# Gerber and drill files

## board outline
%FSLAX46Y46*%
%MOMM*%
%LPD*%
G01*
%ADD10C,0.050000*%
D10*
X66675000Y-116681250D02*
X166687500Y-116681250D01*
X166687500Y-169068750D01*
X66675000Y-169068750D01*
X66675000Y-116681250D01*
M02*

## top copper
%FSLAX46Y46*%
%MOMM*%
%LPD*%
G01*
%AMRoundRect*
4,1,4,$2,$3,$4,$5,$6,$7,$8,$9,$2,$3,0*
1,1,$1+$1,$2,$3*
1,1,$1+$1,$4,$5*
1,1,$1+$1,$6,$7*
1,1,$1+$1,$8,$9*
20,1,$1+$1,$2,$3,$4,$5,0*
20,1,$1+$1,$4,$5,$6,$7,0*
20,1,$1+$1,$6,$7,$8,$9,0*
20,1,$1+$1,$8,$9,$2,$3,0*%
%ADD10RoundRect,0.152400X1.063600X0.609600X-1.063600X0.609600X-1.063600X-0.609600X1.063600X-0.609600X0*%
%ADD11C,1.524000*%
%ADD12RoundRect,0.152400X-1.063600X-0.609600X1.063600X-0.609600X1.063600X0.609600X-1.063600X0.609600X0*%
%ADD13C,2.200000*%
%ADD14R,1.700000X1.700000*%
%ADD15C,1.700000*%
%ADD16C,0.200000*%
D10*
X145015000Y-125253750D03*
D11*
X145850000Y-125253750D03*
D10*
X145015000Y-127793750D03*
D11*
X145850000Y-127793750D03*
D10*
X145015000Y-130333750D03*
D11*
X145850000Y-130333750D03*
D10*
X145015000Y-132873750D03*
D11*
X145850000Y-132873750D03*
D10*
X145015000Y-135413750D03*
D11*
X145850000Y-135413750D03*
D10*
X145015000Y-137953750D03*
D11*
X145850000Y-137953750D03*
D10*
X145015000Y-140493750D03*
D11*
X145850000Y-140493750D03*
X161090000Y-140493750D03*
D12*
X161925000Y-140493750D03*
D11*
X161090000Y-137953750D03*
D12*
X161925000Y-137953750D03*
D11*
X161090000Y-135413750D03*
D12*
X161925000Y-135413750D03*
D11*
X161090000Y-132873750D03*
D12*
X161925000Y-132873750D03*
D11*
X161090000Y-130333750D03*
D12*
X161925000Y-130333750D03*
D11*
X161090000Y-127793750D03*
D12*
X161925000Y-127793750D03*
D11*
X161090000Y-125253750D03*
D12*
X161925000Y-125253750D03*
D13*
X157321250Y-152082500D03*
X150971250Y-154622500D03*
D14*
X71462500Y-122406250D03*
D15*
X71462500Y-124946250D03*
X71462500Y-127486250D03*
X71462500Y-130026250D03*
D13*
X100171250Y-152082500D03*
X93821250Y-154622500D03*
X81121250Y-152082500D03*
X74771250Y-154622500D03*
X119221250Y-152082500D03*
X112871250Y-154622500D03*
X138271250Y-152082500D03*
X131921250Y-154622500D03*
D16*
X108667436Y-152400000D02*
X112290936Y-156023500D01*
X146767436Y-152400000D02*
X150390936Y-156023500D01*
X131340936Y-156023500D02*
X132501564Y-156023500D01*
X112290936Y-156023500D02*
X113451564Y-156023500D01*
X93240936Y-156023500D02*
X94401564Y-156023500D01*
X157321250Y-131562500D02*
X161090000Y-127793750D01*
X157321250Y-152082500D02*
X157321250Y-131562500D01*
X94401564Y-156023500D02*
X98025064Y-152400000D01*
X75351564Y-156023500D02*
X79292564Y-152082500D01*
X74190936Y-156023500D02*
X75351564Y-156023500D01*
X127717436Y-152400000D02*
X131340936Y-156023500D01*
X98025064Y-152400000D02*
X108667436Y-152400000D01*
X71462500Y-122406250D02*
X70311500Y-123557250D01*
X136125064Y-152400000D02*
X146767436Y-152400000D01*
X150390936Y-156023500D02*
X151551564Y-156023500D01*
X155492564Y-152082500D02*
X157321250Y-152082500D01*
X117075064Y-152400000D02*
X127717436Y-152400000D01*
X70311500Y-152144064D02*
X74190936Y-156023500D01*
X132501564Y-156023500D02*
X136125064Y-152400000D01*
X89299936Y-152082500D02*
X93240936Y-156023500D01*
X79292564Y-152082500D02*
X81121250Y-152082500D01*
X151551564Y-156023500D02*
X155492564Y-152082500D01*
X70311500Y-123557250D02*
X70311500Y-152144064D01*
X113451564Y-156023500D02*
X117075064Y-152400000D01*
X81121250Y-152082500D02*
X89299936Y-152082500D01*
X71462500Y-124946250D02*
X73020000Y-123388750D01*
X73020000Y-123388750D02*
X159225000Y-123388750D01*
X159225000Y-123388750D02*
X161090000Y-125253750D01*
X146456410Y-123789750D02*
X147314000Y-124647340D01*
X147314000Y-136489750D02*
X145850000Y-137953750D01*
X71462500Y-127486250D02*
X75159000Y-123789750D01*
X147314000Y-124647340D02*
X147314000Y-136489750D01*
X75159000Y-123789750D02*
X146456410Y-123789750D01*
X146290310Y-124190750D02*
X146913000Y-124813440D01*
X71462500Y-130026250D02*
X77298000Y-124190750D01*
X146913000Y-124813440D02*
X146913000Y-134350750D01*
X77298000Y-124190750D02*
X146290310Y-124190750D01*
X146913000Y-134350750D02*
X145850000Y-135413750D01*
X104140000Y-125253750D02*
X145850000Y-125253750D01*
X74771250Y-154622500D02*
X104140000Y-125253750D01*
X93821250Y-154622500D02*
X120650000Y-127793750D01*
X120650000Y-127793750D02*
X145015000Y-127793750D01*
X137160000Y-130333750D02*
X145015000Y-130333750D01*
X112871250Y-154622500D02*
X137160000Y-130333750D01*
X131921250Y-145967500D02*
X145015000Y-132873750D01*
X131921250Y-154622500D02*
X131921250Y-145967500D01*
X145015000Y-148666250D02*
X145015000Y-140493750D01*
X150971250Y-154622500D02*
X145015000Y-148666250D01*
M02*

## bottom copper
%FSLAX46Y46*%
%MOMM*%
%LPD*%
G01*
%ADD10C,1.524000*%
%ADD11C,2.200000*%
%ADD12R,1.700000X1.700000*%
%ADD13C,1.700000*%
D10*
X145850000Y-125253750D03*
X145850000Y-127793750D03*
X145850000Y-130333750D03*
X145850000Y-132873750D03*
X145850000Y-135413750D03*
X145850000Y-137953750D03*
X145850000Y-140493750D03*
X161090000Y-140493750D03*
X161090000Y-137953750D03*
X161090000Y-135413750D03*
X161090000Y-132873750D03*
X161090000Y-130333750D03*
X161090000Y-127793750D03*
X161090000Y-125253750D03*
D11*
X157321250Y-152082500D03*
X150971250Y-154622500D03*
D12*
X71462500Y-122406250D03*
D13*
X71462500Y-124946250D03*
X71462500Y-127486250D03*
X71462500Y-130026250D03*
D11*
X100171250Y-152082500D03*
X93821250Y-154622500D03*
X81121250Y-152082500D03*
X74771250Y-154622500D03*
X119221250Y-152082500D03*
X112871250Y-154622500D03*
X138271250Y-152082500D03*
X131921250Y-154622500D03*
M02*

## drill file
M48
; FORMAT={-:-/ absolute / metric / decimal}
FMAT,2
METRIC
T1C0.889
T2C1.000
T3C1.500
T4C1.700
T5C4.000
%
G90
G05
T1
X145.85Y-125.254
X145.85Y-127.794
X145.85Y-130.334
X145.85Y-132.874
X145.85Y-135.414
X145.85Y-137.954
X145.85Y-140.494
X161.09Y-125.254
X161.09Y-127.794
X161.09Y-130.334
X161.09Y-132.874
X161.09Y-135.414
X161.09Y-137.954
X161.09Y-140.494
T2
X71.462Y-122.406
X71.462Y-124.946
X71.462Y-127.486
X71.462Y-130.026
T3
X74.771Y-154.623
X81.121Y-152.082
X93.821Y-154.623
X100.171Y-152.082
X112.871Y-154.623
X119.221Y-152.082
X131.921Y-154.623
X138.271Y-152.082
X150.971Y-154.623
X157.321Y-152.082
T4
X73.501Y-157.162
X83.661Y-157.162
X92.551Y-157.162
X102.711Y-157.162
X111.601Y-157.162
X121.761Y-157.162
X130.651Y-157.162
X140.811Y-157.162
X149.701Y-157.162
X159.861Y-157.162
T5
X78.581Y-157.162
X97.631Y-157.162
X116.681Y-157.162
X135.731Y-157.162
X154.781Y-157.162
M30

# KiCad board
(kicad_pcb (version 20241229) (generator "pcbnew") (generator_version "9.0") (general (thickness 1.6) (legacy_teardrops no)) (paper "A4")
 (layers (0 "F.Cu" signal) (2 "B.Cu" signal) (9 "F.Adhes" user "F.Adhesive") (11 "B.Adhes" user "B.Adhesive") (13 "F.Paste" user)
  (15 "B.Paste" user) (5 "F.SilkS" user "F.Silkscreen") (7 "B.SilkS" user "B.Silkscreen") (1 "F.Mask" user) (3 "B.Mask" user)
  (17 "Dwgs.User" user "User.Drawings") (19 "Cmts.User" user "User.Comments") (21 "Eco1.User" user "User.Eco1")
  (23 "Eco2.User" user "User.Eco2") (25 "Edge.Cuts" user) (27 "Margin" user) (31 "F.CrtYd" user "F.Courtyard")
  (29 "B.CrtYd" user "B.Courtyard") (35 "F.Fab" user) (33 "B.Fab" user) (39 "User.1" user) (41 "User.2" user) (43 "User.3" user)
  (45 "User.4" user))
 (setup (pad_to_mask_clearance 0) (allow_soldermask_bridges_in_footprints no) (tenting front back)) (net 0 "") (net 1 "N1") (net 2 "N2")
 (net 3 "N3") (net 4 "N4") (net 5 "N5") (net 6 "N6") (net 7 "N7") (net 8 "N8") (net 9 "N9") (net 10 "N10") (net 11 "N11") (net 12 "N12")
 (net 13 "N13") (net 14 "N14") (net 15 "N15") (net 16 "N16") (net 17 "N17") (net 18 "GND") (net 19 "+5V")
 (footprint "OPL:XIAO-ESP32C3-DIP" (layer "F.Cu") (at 153.59 132.87375)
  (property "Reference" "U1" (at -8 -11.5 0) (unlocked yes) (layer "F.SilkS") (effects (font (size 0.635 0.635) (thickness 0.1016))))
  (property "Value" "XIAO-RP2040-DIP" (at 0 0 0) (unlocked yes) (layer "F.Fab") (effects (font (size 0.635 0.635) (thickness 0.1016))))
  (pad "1" smd roundrect (at -8.575 -7.62 180) (size 2.432 1.524) (layers "F.Cu" "F.Mask") (roundrect_rratio 0.1) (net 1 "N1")
   (thermal_bridge_angle 45))
  (pad "1" thru_hole circle (at -7.74 -7.62 180) (size 1.524 1.524) (drill 0.889) (layers "*.Cu" "*.Mask") (remove_unused_layers no)
   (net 1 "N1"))
  (pad "2" smd roundrect (at -8.575 -5.08 180) (size 2.432 1.524) (layers "F.Cu" "F.Mask") (roundrect_rratio 0.1) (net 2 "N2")
   (thermal_bridge_angle 45))
  (pad "2" thru_hole circle (at -7.74 -5.08 180) (size 1.524 1.524) (drill 0.889) (layers "*.Cu" "*.Mask") (remove_unused_layers no)
   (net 2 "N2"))
  (pad "3" smd roundrect (at -8.575 -2.54 180) (size 2.432 1.524) (layers "F.Cu" "F.Mask") (roundrect_rratio 0.1) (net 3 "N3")
   (thermal_bridge_angle 45))
  (pad "3" thru_hole circle (at -7.74 -2.54 180) (size 1.524 1.524) (drill 0.889) (layers "*.Cu" "*.Mask") (remove_unused_layers no)
   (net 3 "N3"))
  (pad "4" smd roundrect (at -8.575 0 180) (size 2.432 1.524) (layers "F.Cu" "F.Mask") (roundrect_rratio 0.1) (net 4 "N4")
   (thermal_bridge_angle 45))
  (pad "4" thru_hole circle (at -7.74 0 180) (size 1.524 1.524) (drill 0.889) (layers "*.Cu" "*.Mask") (remove_unused_layers no)
   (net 4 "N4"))
  (pad "5" smd roundrect (at -8.575 2.54 180) (size 2.432 1.524) (layers "F.Cu" "F.Mask") (roundrect_rratio 0.1) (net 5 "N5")
   (thermal_bridge_angle 45))
  (pad "5" thru_hole circle (at -7.74 2.54 180) (size 1.524 1.524) (drill 0.889) (layers "*.Cu" "*.Mask") (remove_unused_layers no)
   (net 5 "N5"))
  (pad "6" smd roundrect (at -8.575 5.08 180) (size 2.432 1.524) (layers "F.Cu" "F.Mask") (roundrect_rratio 0.1) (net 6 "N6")
   (thermal_bridge_angle 45))
  (pad "6" thru_hole circle (at -7.74 5.08 180) (size 1.524 1.524) (drill 0.889) (layers "*.Cu" "*.Mask") (remove_unused_layers no)
   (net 6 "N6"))
  (pad "7" smd roundrect (at -8.575 7.62 180) (size 2.432 1.524) (layers "F.Cu" "F.Mask") (roundrect_rratio 0.1) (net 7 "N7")
   (thermal_bridge_angle 45))
  (pad "7" thru_hole circle (at -7.74 7.62 180) (size 1.524 1.524) (drill 0.889) (layers "*.Cu" "*.Mask") (remove_unused_layers no)
   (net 7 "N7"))
  (pad "8" thru_hole circle (at 7.5 7.62) (size 1.524 1.524) (drill 0.889) (layers "*.Cu" "*.Mask") (remove_unused_layers no) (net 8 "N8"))
  (pad "8" smd roundrect (at 8.335 7.62) (size 2.432 1.524) (layers "F.Cu" "F.Mask") (roundrect_rratio 0.1) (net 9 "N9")
   (thermal_bridge_angle 45))
  (pad "9" thru_hole circle (at 7.5 5.08) (size 1.524 1.524) (drill 0.889) (layers "*.Cu" "*.Mask") (remove_unused_layers no) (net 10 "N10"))
  (pad "9" smd roundrect (at 8.335 5.08) (size 2.432 1.524) (layers "F.Cu" "F.Mask") (roundrect_rratio 0.1) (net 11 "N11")
   (thermal_bridge_angle 45))
  (pad "10" thru_hole circle (at 7.5 2.54) (size 1.524 1.524) (drill 0.889) (layers "*.Cu" "*.Mask") (remove_unused_layers no)
   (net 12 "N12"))
  (pad "10" smd roundrect (at 8.335 2.54) (size 2.432 1.524) (layers "F.Cu" "F.Mask") (roundrect_rratio 0.1) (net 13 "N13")
   (thermal_bridge_angle 45))
  (pad "11" thru_hole circle (at 7.5 0) (size 1.524 1.524) (drill 0.889) (layers "*.Cu" "*.Mask") (remove_unused_layers no) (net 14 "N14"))
  (pad "11" smd roundrect (at 8.335 0) (size 2.432 1.524) (layers "F.Cu" "F.Mask") (roundrect_rratio 0.1) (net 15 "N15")
   (thermal_bridge_angle 45))
  (pad "12" thru_hole circle (at 7.5 -2.54) (size 1.524 1.524) (drill 0.889) (layers "*.Cu" "*.Mask") (remove_unused_layers no)
   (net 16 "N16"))
  (pad "12" smd roundrect (at 8.335 -2.54) (size 2.432 1.524) (layers "F.Cu" "F.Mask") (roundrect_rratio 0.1) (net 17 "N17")
   (thermal_bridge_angle 45))
  (pad "13" thru_hole circle (at 7.5 -5.08) (size 1.524 1.524) (drill 0.889) (layers "*.Cu" "*.Mask") (remove_unused_layers no)
   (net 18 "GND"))
  (pad "13" smd roundrect (at 8.335 -5.08) (size 2.432 1.524) (layers "F.Cu" "F.Mask") (roundrect_rratio 0.1) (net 18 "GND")
   (thermal_bridge_angle 45))
  (pad "14" thru_hole circle (at 7.5 -7.62) (size 1.524 1.524) (drill 0.889) (layers "*.Cu" "*.Mask") (remove_unused_layers no)
   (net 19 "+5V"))
  (pad "14" smd roundrect (at 8.335 -7.62) (size 2.432 1.524) (layers "F.Cu" "F.Mask") (roundrect_rratio 0.1) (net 19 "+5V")
   (thermal_bridge_angle 45)))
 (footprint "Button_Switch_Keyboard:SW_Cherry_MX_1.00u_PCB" (layer "F.Cu") (at 157.32125 152.0825)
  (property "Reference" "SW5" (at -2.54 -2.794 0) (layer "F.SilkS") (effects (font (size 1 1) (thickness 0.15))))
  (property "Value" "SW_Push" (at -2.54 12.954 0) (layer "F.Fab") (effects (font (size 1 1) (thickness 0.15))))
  (pad "" np_thru_hole circle (at -7.62 5.08) (size 1.7 1.7) (drill 1.7) (layers "*.Cu" "*.Mask"))
  (pad "" np_thru_hole circle (at -2.54 5.08) (size 4 4) (drill 4) (layers "*.Cu" "*.Mask"))
  (pad "" np_thru_hole circle (at 2.54 5.08) (size 1.7 1.7) (drill 1.7) (layers "*.Cu" "*.Mask"))
  (pad "1" thru_hole circle (at 0 0) (size 2.2 2.2) (drill 1.5) (layers "*.Cu" "*.Mask") (remove_unused_layers no) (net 18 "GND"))
  (pad "2" thru_hole circle (at -6.35 2.54) (size 2.2 2.2) (drill 1.5) (layers "*.Cu" "*.Mask") (remove_unused_layers no) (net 7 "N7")))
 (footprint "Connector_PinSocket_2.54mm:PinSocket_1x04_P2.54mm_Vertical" (layer "F.Cu") (at 71.4625 122.40625)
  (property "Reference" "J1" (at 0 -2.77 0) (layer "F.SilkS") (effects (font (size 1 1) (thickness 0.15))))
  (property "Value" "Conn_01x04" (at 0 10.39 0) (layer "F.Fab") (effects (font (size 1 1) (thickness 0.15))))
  (pad "1" thru_hole rect (at 0 0) (size 1.7 1.7) (drill 1) (layers "*.Cu" "*.Mask") (remove_unused_layers no) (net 18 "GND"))
  (pad "2" thru_hole circle (at 0 2.54) (size 1.7 1.7) (drill 1) (layers "*.Cu" "*.Mask") (remove_unused_layers no) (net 19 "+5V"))
  (pad "3" thru_hole circle (at 0 5.08) (size 1.7 1.7) (drill 1) (layers "*.Cu" "*.Mask") (remove_unused_layers no) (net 6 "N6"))
  (pad "4" thru_hole circle (at 0 7.62) (size 1.7 1.7) (drill 1) (layers "*.Cu" "*.Mask") (remove_unused_layers no) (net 5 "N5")))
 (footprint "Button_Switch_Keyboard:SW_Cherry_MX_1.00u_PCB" (layer "F.Cu") (at 100.17125 152.0825)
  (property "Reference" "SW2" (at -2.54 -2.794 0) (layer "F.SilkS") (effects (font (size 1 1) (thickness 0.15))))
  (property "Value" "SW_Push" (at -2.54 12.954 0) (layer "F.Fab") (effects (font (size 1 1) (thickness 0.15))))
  (pad "" np_thru_hole circle (at -7.62 5.08) (size 1.7 1.7) (drill 1.7) (layers "*.Cu" "*.Mask"))
  (pad "" np_thru_hole circle (at -2.54 5.08) (size 4 4) (drill 4) (layers "*.Cu" "*.Mask"))
  (pad "" np_thru_hole circle (at 2.54 5.08) (size 1.7 1.7) (drill 1.7) (layers "*.Cu" "*.Mask"))
  (pad "1" thru_hole circle (at 0 0) (size 2.2 2.2) (drill 1.5) (layers "*.Cu" "*.Mask") (remove_unused_layers no) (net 18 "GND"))
  (pad "2" thru_hole circle (at -6.35 2.54) (size 2.2 2.2) (drill 1.5) (layers "*.Cu" "*.Mask") (remove_unused_layers no) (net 2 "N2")))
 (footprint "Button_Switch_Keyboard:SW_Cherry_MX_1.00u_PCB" (layer "F.Cu") (at 81.12125 152.0825)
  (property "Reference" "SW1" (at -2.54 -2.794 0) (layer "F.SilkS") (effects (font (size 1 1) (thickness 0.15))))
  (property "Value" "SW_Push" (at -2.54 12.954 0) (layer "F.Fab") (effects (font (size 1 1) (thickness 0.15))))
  (pad "" np_thru_hole circle (at -7.62 5.08) (size 1.7 1.7) (drill 1.7) (layers "*.Cu" "*.Mask"))
  (pad "" np_thru_hole circle (at -2.54 5.08) (size 4 4) (drill 4) (layers "*.Cu" "*.Mask"))
  (pad "" np_thru_hole circle (at 2.54 5.08) (size 1.7 1.7) (drill 1.7) (layers "*.Cu" "*.Mask"))
  (pad "1" thru_hole circle (at 0 0) (size 2.2 2.2) (drill 1.5) (layers "*.Cu" "*.Mask") (remove_unused_layers no) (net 18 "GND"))
  (pad "2" thru_hole circle (at -6.35 2.54) (size 2.2 2.2) (drill 1.5) (layers "*.Cu" "*.Mask") (remove_unused_layers no) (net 1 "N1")))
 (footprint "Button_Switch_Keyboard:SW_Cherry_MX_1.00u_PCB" (layer "F.Cu") (at 119.22125 152.0825)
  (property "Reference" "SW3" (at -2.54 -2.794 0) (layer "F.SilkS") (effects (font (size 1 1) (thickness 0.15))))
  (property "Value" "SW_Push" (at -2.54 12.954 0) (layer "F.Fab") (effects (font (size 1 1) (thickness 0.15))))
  (pad "" np_thru_hole circle (at -7.62 5.08) (size 1.7 1.7) (drill 1.7) (layers "*.Cu" "*.Mask"))
  (pad "" np_thru_hole circle (at -2.54 5.08) (size 4 4) (drill 4) (layers "*.Cu" "*.Mask"))
  (pad "" np_thru_hole circle (at 2.54 5.08) (size 1.7 1.7) (drill 1.7) (layers "*.Cu" "*.Mask"))
  (pad "1" thru_hole circle (at 0 0) (size 2.2 2.2) (drill 1.5) (layers "*.Cu" "*.Mask") (remove_unused_layers no) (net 18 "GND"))
  (pad "2" thru_hole circle (at -6.35 2.54) (size 2.2 2.2) (drill 1.5) (layers "*.Cu" "*.Mask") (remove_unused_layers no) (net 3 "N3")))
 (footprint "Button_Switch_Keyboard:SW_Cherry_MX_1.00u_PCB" (layer "F.Cu") (at 138.27125 152.0825)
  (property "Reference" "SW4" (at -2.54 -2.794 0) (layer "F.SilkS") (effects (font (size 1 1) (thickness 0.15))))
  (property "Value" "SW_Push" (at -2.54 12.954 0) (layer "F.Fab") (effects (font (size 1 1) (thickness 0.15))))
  (pad "" np_thru_hole circle (at -7.62 5.08) (size 1.7 1.7) (drill 1.7) (layers "*.Cu" "*.Mask"))
  (pad "" np_thru_hole circle (at -2.54 5.08) (size 4 4) (drill 4) (layers "*.Cu" "*.Mask"))
  (pad "" np_thru_hole circle (at 2.54 5.08) (size 1.7 1.7) (drill 1.7) (layers "*.Cu" "*.Mask"))
  (pad "1" thru_hole circle (at 0 0) (size 2.2 2.2) (drill 1.5) (layers "*.Cu" "*.Mask") (remove_unused_layers no) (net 18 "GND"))
  (pad "2" thru_hole circle (at -6.35 2.54) (size 2.2 2.2) (drill 1.5) (layers "*.Cu" "*.Mask") (remove_unused_layers no) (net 4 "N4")))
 (gr_rect (start 66.675 116.68125) (end 166.6875 169.06875) (stroke (width 0.05) (type default)) (fill no) (layer "Edge.Cuts"))
 (segment (start 108.667436 152.4) (end 112.290936 156.0235) (width 0.2) (layer "F.Cu") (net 18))
 (segment (start 146.767436 152.4) (end 150.390936 156.0235) (width 0.2) (layer "F.Cu") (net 18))
 (segment (start 131.340936 156.0235) (end 132.501564 156.0235) (width 0.2) (layer "F.Cu") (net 18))
 (segment (start 112.290936 156.0235) (end 113.451564 156.0235) (width 0.2) (layer "F.Cu") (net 18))
 (segment (start 93.240936 156.0235) (end 94.401564 156.0235) (width 0.2) (layer "F.Cu") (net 18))
 (segment (start 157.32125 131.5625) (end 161.09 127.79375) (width 0.2) (layer "F.Cu") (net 18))
 (segment (start 157.32125 152.0825) (end 157.32125 131.5625) (width 0.2) (layer "F.Cu") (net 18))
 (segment (start 94.401564 156.0235) (end 98.025064 152.4) (width 0.2) (layer "F.Cu") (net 18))
 (segment (start 75.351564 156.0235) (end 79.292564 152.0825) (width 0.2) (layer "F.Cu") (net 18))
 (segment (start 74.190936 156.0235) (end 75.351564 156.0235) (width 0.2) (layer "F.Cu") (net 18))
 (segment (start 127.717436 152.4) (end 131.340936 156.0235) (width 0.2) (layer "F.Cu") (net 18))
 (segment (start 98.025064 152.4) (end 108.667436 152.4) (width 0.2) (layer "F.Cu") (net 18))
 (segment (start 71.4625 122.40625) (end 70.3115 123.55725) (width 0.2) (layer "F.Cu") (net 18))
 (segment (start 136.125064 152.4) (end 146.767436 152.4) (width 0.2) (layer "F.Cu") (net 18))
 (segment (start 150.390936 156.0235) (end 151.551564 156.0235) (width 0.2) (layer "F.Cu") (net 18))
 (segment (start 155.492564 152.0825) (end 157.32125 152.0825) (width 0.2) (layer "F.Cu") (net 18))
 (segment (start 117.075064 152.4) (end 127.717436 152.4) (width 0.2) (layer "F.Cu") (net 18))
 (segment (start 70.3115 152.144064) (end 74.190936 156.0235) (width 0.2) (layer "F.Cu") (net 18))
 (segment (start 132.501564 156.0235) (end 136.125064 152.4) (width 0.2) (layer "F.Cu") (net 18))
 (segment (start 89.299936 152.0825) (end 93.240936 156.0235) (width 0.2) (layer "F.Cu") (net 18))
 (segment (start 79.292564 152.0825) (end 81.12125 152.0825) (width 0.2) (layer "F.Cu") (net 18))
 (segment (start 151.551564 156.0235) (end 155.492564 152.0825) (width 0.2) (layer "F.Cu") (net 18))
 (segment (start 70.3115 123.55725) (end 70.3115 152.144064) (width 0.2) (layer "F.Cu") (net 18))
 (segment (start 113.451564 156.0235) (end 117.075064 152.4) (width 0.2) (layer "F.Cu") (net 18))
 (segment (start 81.12125 152.0825) (end 89.299936 152.0825) (width 0.2) (layer "F.Cu") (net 18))
 (segment (start 71.4625 124.94625) (end 73.02 123.38875) (width 0.2) (layer "F.Cu") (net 19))
 (segment (start 73.02 123.38875) (end 159.225 123.38875) (width 0.2) (layer "F.Cu") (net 19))
 (segment (start 159.225 123.38875) (end 161.09 125.25375) (width 0.2) (layer "F.Cu") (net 19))
 (segment (start 146.45641 123.78975) (end 147.314 124.64734) (width 0.2) (layer "F.Cu") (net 6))
 (segment (start 147.314 136.48975) (end 145.85 137.95375) (width 0.2) (layer "F.Cu") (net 6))
 (segment (start 71.4625 127.48625) (end 75.159 123.78975) (width 0.2) (layer "F.Cu") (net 6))
 (segment (start 147.314 124.64734) (end 147.314 136.48975) (width 0.2) (layer "F.Cu") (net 6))
 (segment (start 75.159 123.78975) (end 146.45641 123.78975) (width 0.2) (layer "F.Cu") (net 6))
 (segment (start 146.29031 124.19075) (end 146.913 124.81344) (width 0.2) (layer "F.Cu") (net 5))
 (segment (start 71.4625 130.02625) (end 77.298 124.19075) (width 0.2) (layer "F.Cu") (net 5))
 (segment (start 146.913 124.81344) (end 146.913 134.35075) (width 0.2) (layer "F.Cu") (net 5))
 (segment (start 77.298 124.19075) (end 146.29031 124.19075) (width 0.2) (layer "F.Cu") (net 5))
 (segment (start 146.913 134.35075) (end 145.85 135.41375) (width 0.2) (layer "F.Cu") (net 5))
 (segment (start 104.14 125.25375) (end 145.85 125.25375) (width 0.2) (layer "F.Cu") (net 1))
 (segment (start 74.77125 154.6225) (end 104.14 125.25375) (width 0.2) (layer "F.Cu") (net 1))
 (segment (start 93.82125 154.6225) (end 120.65 127.79375) (width 0.2) (layer "F.Cu") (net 2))
 (segment (start 120.65 127.79375) (end 145.015 127.79375) (width 0.2) (layer "F.Cu") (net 2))
 (segment (start 137.16 130.33375) (end 145.015 130.33375) (width 0.2) (layer "F.Cu") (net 3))
 (segment (start 112.87125 154.6225) (end 137.16 130.33375) (width 0.2) (layer "F.Cu") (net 3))
 (segment (start 131.92125 145.9675) (end 145.015 132.87375) (width 0.2) (layer "F.Cu") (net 4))
 (segment (start 131.92125 154.6225) (end 131.92125 145.9675) (width 0.2) (layer "F.Cu") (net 4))
 (segment (start 145.015 148.66625) (end 145.015 140.49375) (width 0.2) (layer "F.Cu") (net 7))
 (segment (start 150.97125 154.6225) (end 145.015 148.66625) (width 0.2) (layer "F.Cu") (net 7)))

